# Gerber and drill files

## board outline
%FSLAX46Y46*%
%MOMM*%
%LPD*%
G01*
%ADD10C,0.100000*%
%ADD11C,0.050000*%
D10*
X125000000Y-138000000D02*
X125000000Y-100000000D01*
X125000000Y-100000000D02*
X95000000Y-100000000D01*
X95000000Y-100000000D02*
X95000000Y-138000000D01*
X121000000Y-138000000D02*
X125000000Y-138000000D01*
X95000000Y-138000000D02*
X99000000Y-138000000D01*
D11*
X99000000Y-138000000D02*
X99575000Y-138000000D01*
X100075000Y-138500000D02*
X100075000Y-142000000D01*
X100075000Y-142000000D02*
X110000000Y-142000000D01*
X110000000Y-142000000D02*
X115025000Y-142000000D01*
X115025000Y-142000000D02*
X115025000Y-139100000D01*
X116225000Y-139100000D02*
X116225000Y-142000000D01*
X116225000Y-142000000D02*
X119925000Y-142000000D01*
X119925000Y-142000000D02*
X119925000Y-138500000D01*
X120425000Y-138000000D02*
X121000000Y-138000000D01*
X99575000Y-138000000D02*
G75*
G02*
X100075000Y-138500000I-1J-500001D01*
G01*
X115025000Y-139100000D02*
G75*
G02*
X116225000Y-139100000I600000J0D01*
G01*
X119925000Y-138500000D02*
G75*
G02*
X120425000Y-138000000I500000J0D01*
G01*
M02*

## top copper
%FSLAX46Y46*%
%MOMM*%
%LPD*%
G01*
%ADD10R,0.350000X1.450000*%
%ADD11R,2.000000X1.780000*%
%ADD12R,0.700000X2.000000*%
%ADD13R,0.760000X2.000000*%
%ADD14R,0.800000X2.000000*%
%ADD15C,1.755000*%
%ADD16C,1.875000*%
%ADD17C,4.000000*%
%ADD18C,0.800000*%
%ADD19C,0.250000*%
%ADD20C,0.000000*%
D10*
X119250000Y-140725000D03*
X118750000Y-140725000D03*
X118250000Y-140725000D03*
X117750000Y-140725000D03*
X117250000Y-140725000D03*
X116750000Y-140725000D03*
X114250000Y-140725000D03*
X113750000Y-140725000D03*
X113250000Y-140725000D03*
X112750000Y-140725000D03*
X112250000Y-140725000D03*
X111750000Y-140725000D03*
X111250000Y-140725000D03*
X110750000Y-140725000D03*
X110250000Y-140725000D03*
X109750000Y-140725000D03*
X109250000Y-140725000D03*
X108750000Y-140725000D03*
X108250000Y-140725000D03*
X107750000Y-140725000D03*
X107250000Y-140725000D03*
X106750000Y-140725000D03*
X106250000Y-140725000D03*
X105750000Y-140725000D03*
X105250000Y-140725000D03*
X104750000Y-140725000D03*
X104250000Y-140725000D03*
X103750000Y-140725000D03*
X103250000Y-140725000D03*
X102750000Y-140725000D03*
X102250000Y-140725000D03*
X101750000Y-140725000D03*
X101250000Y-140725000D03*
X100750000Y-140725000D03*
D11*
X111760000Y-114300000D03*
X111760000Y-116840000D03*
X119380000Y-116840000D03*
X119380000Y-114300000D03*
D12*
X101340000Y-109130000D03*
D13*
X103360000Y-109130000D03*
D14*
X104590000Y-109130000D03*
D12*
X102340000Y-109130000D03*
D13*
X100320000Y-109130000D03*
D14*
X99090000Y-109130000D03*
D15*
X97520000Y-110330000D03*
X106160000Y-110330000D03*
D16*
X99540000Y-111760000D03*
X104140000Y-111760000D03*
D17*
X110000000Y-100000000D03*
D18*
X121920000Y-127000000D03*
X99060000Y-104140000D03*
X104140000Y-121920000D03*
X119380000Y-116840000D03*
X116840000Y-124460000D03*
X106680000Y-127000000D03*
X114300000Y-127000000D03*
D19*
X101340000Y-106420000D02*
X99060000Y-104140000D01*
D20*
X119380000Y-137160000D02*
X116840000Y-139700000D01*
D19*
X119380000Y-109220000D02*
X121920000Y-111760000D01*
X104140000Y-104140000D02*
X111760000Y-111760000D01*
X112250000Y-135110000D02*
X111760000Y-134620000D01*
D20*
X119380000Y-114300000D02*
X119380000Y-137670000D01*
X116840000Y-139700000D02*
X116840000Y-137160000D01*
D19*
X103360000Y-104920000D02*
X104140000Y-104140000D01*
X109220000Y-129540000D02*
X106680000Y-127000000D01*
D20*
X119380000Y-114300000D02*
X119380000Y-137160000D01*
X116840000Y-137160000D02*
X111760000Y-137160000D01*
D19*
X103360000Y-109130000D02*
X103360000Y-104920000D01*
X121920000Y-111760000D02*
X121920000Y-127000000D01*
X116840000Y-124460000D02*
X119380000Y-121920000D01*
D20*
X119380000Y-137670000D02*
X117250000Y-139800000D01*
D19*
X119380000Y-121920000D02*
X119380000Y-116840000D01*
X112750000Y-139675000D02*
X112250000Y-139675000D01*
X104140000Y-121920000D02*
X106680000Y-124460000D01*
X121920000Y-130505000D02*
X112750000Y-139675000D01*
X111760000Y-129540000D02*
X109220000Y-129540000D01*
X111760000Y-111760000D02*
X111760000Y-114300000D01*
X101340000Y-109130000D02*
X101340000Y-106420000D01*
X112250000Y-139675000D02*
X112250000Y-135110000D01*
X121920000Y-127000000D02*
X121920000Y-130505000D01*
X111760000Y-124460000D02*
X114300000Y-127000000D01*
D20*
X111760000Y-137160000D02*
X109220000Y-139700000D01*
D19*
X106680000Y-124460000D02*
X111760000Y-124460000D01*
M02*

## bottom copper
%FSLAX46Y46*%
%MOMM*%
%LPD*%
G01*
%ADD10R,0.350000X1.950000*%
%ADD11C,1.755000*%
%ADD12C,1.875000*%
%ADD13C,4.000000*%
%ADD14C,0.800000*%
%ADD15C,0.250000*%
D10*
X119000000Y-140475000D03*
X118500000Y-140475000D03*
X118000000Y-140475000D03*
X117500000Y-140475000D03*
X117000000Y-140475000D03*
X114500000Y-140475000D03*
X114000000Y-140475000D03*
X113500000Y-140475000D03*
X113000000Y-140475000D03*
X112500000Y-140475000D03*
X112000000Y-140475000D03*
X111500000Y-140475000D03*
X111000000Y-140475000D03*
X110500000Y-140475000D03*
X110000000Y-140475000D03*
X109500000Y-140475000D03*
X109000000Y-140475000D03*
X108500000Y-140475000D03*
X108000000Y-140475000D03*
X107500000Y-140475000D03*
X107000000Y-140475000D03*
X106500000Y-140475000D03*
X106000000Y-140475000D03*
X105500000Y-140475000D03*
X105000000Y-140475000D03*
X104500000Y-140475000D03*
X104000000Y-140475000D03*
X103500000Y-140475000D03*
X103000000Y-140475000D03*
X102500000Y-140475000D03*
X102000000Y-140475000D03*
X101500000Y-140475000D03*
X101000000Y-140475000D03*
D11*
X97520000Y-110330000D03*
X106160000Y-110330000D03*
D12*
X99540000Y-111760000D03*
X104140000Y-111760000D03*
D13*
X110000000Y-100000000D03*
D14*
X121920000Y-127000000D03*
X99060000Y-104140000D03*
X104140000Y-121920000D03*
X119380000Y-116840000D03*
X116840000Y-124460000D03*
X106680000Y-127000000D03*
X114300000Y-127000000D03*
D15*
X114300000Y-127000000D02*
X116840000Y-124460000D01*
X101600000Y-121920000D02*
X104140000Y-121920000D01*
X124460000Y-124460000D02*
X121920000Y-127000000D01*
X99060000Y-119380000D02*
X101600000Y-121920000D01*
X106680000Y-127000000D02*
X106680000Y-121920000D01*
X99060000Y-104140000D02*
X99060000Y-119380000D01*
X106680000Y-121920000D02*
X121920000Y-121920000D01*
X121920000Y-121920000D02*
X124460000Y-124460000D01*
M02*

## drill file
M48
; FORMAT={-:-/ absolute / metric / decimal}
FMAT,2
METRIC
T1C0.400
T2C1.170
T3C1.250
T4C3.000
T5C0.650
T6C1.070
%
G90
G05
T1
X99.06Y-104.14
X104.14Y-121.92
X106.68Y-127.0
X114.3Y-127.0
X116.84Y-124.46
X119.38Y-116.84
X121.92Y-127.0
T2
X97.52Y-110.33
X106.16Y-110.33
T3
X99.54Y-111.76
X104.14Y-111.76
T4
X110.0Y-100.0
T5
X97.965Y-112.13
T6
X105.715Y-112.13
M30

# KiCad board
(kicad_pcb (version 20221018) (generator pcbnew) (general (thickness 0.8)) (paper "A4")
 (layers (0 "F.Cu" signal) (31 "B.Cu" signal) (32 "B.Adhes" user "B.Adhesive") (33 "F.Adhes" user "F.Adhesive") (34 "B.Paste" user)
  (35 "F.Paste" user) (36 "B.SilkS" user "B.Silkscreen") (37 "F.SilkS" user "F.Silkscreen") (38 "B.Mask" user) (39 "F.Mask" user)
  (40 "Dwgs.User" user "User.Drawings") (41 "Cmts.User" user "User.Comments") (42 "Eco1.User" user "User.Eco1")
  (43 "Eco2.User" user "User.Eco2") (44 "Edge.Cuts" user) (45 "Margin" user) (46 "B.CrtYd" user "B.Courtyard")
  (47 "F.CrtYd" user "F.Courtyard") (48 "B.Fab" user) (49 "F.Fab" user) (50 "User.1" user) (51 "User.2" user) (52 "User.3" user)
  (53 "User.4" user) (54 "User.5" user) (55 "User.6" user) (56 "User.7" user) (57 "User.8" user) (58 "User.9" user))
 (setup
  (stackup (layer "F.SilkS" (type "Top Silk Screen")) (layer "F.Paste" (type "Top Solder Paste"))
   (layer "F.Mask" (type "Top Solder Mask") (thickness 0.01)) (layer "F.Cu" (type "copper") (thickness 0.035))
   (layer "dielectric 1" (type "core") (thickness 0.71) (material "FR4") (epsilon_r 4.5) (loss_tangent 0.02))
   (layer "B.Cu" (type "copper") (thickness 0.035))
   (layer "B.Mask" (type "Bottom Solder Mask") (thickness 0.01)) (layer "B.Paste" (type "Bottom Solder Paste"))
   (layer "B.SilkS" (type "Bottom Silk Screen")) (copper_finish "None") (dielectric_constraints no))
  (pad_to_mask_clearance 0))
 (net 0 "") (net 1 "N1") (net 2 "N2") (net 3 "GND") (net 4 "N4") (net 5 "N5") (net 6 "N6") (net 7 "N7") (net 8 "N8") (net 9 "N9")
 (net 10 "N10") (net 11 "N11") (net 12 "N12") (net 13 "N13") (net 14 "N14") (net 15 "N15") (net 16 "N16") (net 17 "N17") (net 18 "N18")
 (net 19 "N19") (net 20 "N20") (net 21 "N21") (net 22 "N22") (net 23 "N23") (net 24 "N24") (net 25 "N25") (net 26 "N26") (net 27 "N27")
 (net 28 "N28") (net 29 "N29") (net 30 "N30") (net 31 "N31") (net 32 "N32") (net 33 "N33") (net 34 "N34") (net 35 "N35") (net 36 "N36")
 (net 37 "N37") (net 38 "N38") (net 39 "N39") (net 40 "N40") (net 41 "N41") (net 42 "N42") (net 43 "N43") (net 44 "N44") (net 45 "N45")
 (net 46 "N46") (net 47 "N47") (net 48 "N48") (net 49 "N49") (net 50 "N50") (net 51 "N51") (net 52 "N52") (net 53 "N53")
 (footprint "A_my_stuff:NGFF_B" (layer "F.Cu") (at 110 142)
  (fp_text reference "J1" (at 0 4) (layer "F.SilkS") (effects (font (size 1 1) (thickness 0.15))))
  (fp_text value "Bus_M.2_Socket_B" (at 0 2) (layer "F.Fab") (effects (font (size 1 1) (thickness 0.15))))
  (fp_line (start -11 -4) (end -10.425 -4) (stroke (width 0.05) (type solid)) (layer "Edge.Cuts"))
  (fp_line (start -9.925 -3.5) (end -9.925 0) (stroke (width 0.05) (type solid)) (layer "Edge.Cuts"))
  (fp_line (start -9.925 0) (end 0 0) (stroke (width 0.05) (type solid)) (layer "Edge.Cuts"))
  (fp_line (start 0 0) (end 5.025 0) (stroke (width 0.05) (type solid)) (layer "Edge.Cuts"))
  (fp_line (start 5.025 0) (end 5.025 -2.9) (stroke (width 0.05) (type solid)) (layer "Edge.Cuts"))
  (fp_line (start 6.225 -2.9) (end 6.225 0) (stroke (width 0.05) (type solid)) (layer "Edge.Cuts"))
  (fp_line (start 6.225 0) (end 9.925 0) (stroke (width 0.05) (type solid)) (layer "Edge.Cuts"))
  (fp_line (start 9.925 0) (end 9.925 -3.5) (stroke (width 0.05) (type solid)) (layer "Edge.Cuts"))
  (fp_line (start 10.425 -4) (end 11 -4) (stroke (width 0.05) (type solid)) (layer "Edge.Cuts"))
  (fp_arc (start -10.425 -4) (mid -10.071447 -3.853553) (end -9.925 -3.5) (stroke (width 0.05) (type solid)) (layer "Edge.Cuts"))
  (fp_arc (start 5.025 -2.9) (mid 5.625 -3.5) (end 6.225 -2.9) (stroke (width 0.05) (type solid)) (layer "Edge.Cuts"))
  (fp_arc (start 9.925 -3.5) (mid 10.071447 -3.853553) (end 10.425 -4) (stroke (width 0.05) (type solid)) (layer "Edge.Cuts"))
  (pad "1" smd rect (at 9.25 -1.275) (size 0.35 1.45) (layers "F.Cu") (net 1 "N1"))
  (pad "2" smd rect (at 9 -1.525) (size 0.35 1.95) (layers "B.Cu") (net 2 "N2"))
  (pad "3" smd rect (at 8.75 -1.275) (size 0.35 1.45) (layers "F.Cu") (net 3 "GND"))
  (pad "4" smd rect (at 8.5 -1.525) (size 0.35 1.95) (layers "B.Cu") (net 2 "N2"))
  (pad "5" smd rect (at 8.25 -1.275) (size 0.35 1.45) (layers "F.Cu") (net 3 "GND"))
  (pad "6" smd rect (at 8 -1.525) (size 0.35 1.95) (layers "B.Cu") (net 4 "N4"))
  (pad "7" smd rect (at 7.75 -1.275) (size 0.35 1.45) (layers "F.Cu") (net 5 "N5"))
  (pad "8" smd rect (at 7.5 -1.525) (size 0.35 1.95) (layers "B.Cu") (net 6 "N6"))
  (pad "9" smd rect (at 7.25 -1.275) (size 0.35 1.45) (layers "F.Cu") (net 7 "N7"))
  (pad "10" smd rect (at 7 -1.525) (size 0.35 1.95) (layers "B.Cu") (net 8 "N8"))
  (pad "11" smd rect (at 6.75 -1.275) (size 0.35 1.45) (layers "F.Cu") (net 3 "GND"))
  (pad "20" smd rect (at 4.5 -1.525) (size 0.35 1.95) (layers "B.Cu") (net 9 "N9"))
  (pad "21" smd rect (at 4.25 -1.275) (size 0.35 1.45) (layers "F.Cu") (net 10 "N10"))
  (pad "22" smd rect (at 4 -1.525) (size 0.35 1.95) (layers "B.Cu") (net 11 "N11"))
  (pad "23" smd rect (at 3.75 -1.275) (size 0.35 1.45) (layers "F.Cu") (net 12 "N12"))
  (pad "24" smd rect (at 3.5 -1.525) (size 0.35 1.95) (layers "B.Cu") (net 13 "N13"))
  (pad "25" smd rect (at 3.25 -1.275) (size 0.35 1.45) (layers "F.Cu") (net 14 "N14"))
  (pad "26" smd rect (at 3 -1.525) (size 0.35 1.95) (layers "B.Cu") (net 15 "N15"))
  (pad "27" smd rect (at 2.75 -1.275) (size 0.35 1.45) (layers "F.Cu") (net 3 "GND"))
  (pad "28" smd rect (at 2.5 -1.525) (size 0.35 1.95) (layers "B.Cu") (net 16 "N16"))
  (pad "29" smd rect (at 2.25 -1.275) (size 0.35 1.45) (layers "F.Cu") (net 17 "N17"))
  (pad "30" smd rect (at 2 -1.525) (size 0.35 1.95) (layers "B.Cu") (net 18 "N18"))
  (pad "31" smd rect (at 1.75 -1.275) (size 0.35 1.45) (layers "F.Cu") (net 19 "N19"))
  (pad "32" smd rect (at 1.5 -1.525) (size 0.35 1.95) (layers "B.Cu") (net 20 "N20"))
  (pad "33" smd rect (at 1.25 -1.275) (size 0.35 1.45) (layers "F.Cu") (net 3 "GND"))
  (pad "34" smd rect (at 1 -1.525) (size 0.35 1.95) (layers "B.Cu") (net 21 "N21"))
  (pad "35" smd rect (at 0.75 -1.275) (size 0.35 1.45) (layers "F.Cu") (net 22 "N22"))
  (pad "36" smd rect (at 0.5 -1.525) (size 0.35 1.95) (layers "B.Cu") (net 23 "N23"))
  (pad "37" smd rect (at 0.25 -1.275) (size 0.35 1.45) (layers "F.Cu") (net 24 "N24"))
  (pad "38" smd rect (at 0 -1.525) (size 0.35 1.95) (layers "B.Cu") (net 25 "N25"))
  (pad "39" smd rect (at -0.25 -1.275) (size 0.35 1.45) (layers "F.Cu") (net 3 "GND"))
  (pad "40" smd rect (at -0.5 -1.525) (size 0.35 1.95) (layers "B.Cu") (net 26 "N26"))
  (pad "41" smd rect (at -0.75 -1.275) (size 0.35 1.45) (layers "F.Cu") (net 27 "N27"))
  (pad "42" smd rect (at -1 -1.525) (size 0.35 1.95) (layers "B.Cu") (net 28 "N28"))
  (pad "43" smd rect (at -1.25 -1.275) (size 0.35 1.45) (layers "F.Cu") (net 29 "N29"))
  (pad "44" smd rect (at -1.5 -1.525) (size 0.35 1.95) (layers "B.Cu") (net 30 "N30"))
  (pad "45" smd rect (at -1.75 -1.275) (size 0.35 1.45) (layers "F.Cu") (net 3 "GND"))
  (pad "46" smd rect (at -2 -1.525) (size 0.35 1.95) (layers "B.Cu") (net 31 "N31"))
  (pad "47" smd rect (at -2.25 -1.275) (size 0.35 1.45) (layers "F.Cu") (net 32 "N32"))
  (pad "48" smd rect (at -2.5 -1.525) (size 0.35 1.95) (layers "B.Cu") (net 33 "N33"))
  (pad "49" smd rect (at -2.75 -1.275) (size 0.35 1.45) (layers "F.Cu") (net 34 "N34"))
  (pad "50" smd rect (at -3 -1.525) (size 0.35 1.95) (layers "B.Cu") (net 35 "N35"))
  (pad "51" smd rect (at -3.25 -1.275) (size 0.35 1.45) (layers "F.Cu") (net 3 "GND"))
  (pad "52" smd rect (at -3.5 -1.525) (size 0.35 1.95) (layers "B.Cu") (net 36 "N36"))
  (pad "53" smd rect (at -3.75 -1.275) (size 0.35 1.45) (layers "F.Cu") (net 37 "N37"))
  (pad "54" smd rect (at -4 -1.525) (size 0.35 1.95) (layers "B.Cu") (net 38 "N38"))
  (pad "55" smd rect (at -4.25 -1.275) (size 0.35 1.45) (layers "F.Cu") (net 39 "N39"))
  (pad "56" smd rect (at -4.5 -1.525) (size 0.35 1.95) (layers "B.Cu") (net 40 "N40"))
  (pad "57" smd rect (at -4.75 -1.275) (size 0.35 1.45) (layers "F.Cu") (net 3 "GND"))
  (pad "58" smd rect (at -5 -1.525) (size 0.35 1.95) (layers "B.Cu") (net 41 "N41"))
  (pad "59" smd rect (at -5.25 -1.275) (size 0.35 1.45) (layers "F.Cu") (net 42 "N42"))
  (pad "60" smd rect (at -5.5 -1.525) (size 0.35 1.95) (layers "B.Cu") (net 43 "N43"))
  (pad "61" smd rect (at -5.75 -1.275) (size 0.35 1.45) (layers "F.Cu") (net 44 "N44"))
  (pad "62" smd rect (at -6 -1.525) (size 0.35 1.95) (layers "B.Cu") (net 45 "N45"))
  (pad "63" smd rect (at -6.25 -1.275) (size 0.35 1.45) (layers "F.Cu") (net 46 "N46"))
  (pad "64" smd rect (at -6.5 -1.525) (size 0.35 1.95) (layers "B.Cu") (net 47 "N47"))
  (pad "65" smd rect (at -6.75 -1.275) (size 0.35 1.45) (layers "F.Cu") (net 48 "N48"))
  (pad "66" smd rect (at -7 -1.525) (size 0.35 1.95) (layers "B.Cu") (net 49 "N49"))
  (pad "67" smd rect (at -7.25 -1.275) (size 0.35 1.45) (layers "F.Cu") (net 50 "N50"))
  (pad "68" smd rect (at -7.5 -1.525) (size 0.35 1.95) (layers "B.Cu") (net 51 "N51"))
  (pad "69" smd rect (at -7.75 -1.275) (size 0.35 1.45) (layers "F.Cu") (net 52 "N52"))
  (pad "70" smd rect (at -8 -1.525) (size 0.35 1.95) (layers "B.Cu") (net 2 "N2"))
  (pad "71" smd rect (at -8.25 -1.275) (size 0.35 1.45) (layers "F.Cu") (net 3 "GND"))
  (pad "72" smd rect (at -8.5 -1.525) (size 0.35 1.95) (layers "B.Cu") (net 2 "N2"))
  (pad "73" smd rect (at -8.75 -1.275) (size 0.35 1.45) (layers "F.Cu") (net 3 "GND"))
  (pad "74" smd rect (at -9 -1.525) (size 0.35 1.95) (layers "B.Cu") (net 2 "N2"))
  (pad "75" smd rect (at -9.25 -1.275) (size 0.35 1.45) (layers "F.Cu") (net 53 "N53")))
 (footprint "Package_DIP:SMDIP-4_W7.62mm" (layer "F.Cu") (at 115.57 115.57)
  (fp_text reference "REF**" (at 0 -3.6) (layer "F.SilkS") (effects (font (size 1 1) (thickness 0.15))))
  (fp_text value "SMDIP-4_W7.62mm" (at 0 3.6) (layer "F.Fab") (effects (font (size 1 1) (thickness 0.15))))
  (pad "1" smd rect (at -3.81 -1.27) (size 2 1.78) (layers "F.Cu" "F.Paste" "F.Mask"))
  (pad "2" smd rect (at -3.81 1.27) (size 2 1.78) (layers "F.Cu" "F.Paste" "F.Mask"))
  (pad "3" smd rect (at 3.81 1.27) (size 2 1.78) (layers "F.Cu" "F.Paste" "F.Mask"))
  (pad "4" smd rect (at 3.81 -1.27) (size 2 1.78) (layers "F.Cu" "F.Paste" "F.Mask")))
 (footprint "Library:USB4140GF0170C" (layer "F.Cu") (at 101.84 110.58)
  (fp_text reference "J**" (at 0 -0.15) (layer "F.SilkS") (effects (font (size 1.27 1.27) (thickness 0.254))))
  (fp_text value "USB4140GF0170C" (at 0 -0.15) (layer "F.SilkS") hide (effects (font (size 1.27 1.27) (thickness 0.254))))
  (pad "" np_thru_hole circle (at -3.875 1.55) (size 0.65 0.65) (drill 0.65) (layers "*.Cu" "*.Mask"))
  (pad "" np_thru_hole circle (at 3.875 1.55) (size 1.07 1.07) (drill 1.07) (layers "*.Cu" "*.Mask"))
  (pad "A5" smd rect (at -0.5 -1.45) (size 0.7 2) (layers "F.Cu" "F.Paste" "F.Mask"))
  (pad "A9" smd rect (at 1.52 -1.45) (size 0.76 2) (layers "F.Cu" "F.Paste" "F.Mask"))
  (pad "A12" smd rect (at 2.75 -1.45) (size 0.8 2) (layers "F.Cu" "F.Paste" "F.Mask"))
  (pad "B5" smd rect (at 0.5 -1.45) (size 0.7 2) (layers "F.Cu" "F.Paste" "F.Mask"))
  (pad "B9" smd rect (at -1.52 -1.45) (size 0.76 2) (layers "F.Cu" "F.Paste" "F.Mask"))
  (pad "B12" smd rect (at -2.75 -1.45) (size 0.8 2) (layers "F.Cu" "F.Paste" "F.Mask"))
  (pad "MH1" thru_hole circle (at -4.32 -0.25) (size 1.755 1.755) (drill 1.17) (layers "*.Cu" "*.Mask"))
  (pad "MH2" thru_hole circle (at 4.32 -0.25) (size 1.755 1.755) (drill 1.17) (layers "*.Cu" "*.Mask"))
  (pad "MH3" thru_hole circle (at -2.3 1.18) (size 1.875 1.875) (drill 1.25) (layers "*.Cu" "*.Mask"))
  (pad "MH4" thru_hole circle (at 2.3 1.18) (size 1.875 1.875) (drill 1.25) (layers "*.Cu" "*.Mask")))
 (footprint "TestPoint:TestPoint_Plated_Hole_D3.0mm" (layer "F.Cu") (at 110 100)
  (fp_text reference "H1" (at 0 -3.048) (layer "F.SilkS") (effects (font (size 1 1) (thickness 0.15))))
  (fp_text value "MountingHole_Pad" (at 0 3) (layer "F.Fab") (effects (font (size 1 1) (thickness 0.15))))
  (pad "1" thru_hole circle (at 0 0) (size 4 4) (drill 3) (layers "*.Cu" "*.Mask") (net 3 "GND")))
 (gr_line (start 125 138) (end 125 100) (stroke (width 0.1) (type default)) (layer "Edge.Cuts"))
 (gr_line (start 125 100) (end 95 100) (stroke (width 0.1) (type default)) (layer "Edge.Cuts"))
 (gr_line (start 95 100) (end 95 138) (stroke (width 0.1) (type default)) (layer "Edge.Cuts"))
 (gr_line (start 121 138) (end 125 138) (stroke (width 0.1) (type default)) (layer "Edge.Cuts"))
 (gr_line (start 95 138) (end 99 138) (stroke (width 0.1) (type default)) (layer "Edge.Cuts"))
 (segment (start 101.34 106.42) (end 99.06 104.14) (width 0.25) (layer "F.Cu") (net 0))
 (segment (start 119.38 137.16) (end 116.84 139.7) (width 0) (layer "F.Cu") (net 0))
 (segment (start 119.38 109.22) (end 121.92 111.76) (width 0.25) (layer "F.Cu") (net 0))
 (segment (start 104.14 104.14) (end 111.76 111.76) (width 0.25) (layer "F.Cu") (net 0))
 (segment (start 112.25 135.11) (end 111.76 134.62) (width 0.25) (layer "F.Cu") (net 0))
 (segment (start 119.38 114.3) (end 119.38 137.67) (width 0) (layer "F.Cu") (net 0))
 (segment (start 116.84 139.7) (end 116.84 137.16) (width 0) (layer "F.Cu") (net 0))
 (segment (start 103.36 104.92) (end 104.14 104.14) (width 0.25) (layer "F.Cu") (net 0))
 (segment (start 109.22 129.54) (end 106.68 127) (width 0.25) (layer "F.Cu") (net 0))
 (segment (start 119.38 114.3) (end 119.38 137.16) (width 0) (layer "F.Cu") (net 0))
 (segment (start 116.84 137.16) (end 111.76 137.16) (width 0) (layer "F.Cu") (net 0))
 (segment (start 103.36 109.13) (end 103.36 104.92) (width 0.25) (layer "F.Cu") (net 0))
 (segment (start 121.92 111.76) (end 121.92 127) (width 0.25) (layer "F.Cu") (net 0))
 (segment (start 116.84 124.46) (end 119.38 121.92) (width 0.25) (layer "F.Cu") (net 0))
 (segment (start 119.38 137.67) (end 117.25 139.8) (width 0) (layer "F.Cu") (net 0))
 (segment (start 119.38 121.92) (end 119.38 116.84) (width 0.25) (layer "F.Cu") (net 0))
 (segment (start 112.75 139.675) (end 112.25 139.675) (width 0.25) (layer "F.Cu") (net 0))
 (segment (start 104.14 121.92) (end 106.68 124.46) (width 0.25) (layer "F.Cu") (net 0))
 (segment (start 121.92 130.505) (end 112.75 139.675) (width 0.25) (layer "F.Cu") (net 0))
 (segment (start 111.76 129.54) (end 109.22 129.54) (width 0.25) (layer "F.Cu") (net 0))
 (segment (start 111.76 111.76) (end 111.76 114.3) (width 0.25) (layer "F.Cu") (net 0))
 (segment (start 101.34 109.13) (end 101.34 106.42) (width 0.25) (layer "F.Cu") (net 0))
 (segment (start 112.25 139.675) (end 112.25 135.11) (width 0.25) (layer "F.Cu") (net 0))
 (segment (start 121.92 127) (end 121.92 130.505) (width 0.25) (layer "F.Cu") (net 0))
 (segment (start 111.76 124.46) (end 114.3 127) (width 0.25) (layer "F.Cu") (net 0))
 (segment (start 111.76 137.16) (end 109.22 139.7) (width 0) (layer "F.Cu") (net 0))
 (segment (start 106.68 124.46) (end 111.76 124.46) (width 0.25) (layer "F.Cu") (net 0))
 (via (at 121.92 127) (size 0.8) (drill 0.4) (layers "F.Cu" "B.Cu") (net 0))
 (via (at 99.06 104.14) (size 0.8) (drill 0.4) (layers "F.Cu" "B.Cu") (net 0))
 (via (at 104.14 121.92) (size 0.8) (drill 0.4) (layers "F.Cu" "B.Cu") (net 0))
 (via (at 119.38 116.84) (size 0.8) (drill 0.4) (layers "F.Cu" "B.Cu") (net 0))
 (via (at 116.84 124.46) (size 0.8) (drill 0.4) (layers "F.Cu" "B.Cu") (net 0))
 (via (at 106.68 127) (size 0.8) (drill 0.4) (layers "F.Cu" "B.Cu") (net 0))
 (via (at 114.3 127) (size 0.8) (drill 0.4) (layers "F.Cu" "B.Cu") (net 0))
 (segment (start 114.3 127) (end 116.84 124.46) (width 0.25) (layer "B.Cu") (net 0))
 (segment (start 101.6 121.92) (end 104.14 121.92) (width 0.25) (layer "B.Cu") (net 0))
 (segment (start 124.46 124.46) (end 121.92 127) (width 0.25) (layer "B.Cu") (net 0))
 (segment (start 99.06 119.38) (end 101.6 121.92) (width 0.25) (layer "B.Cu") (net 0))
 (segment (start 106.68 127) (end 106.68 121.92) (width 0.25) (layer "B.Cu") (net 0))
 (segment (start 99.06 104.14) (end 99.06 119.38) (width 0.25) (layer "B.Cu") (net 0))
 (segment (start 106.68 121.92) (end 121.92 121.92) (width 0.25) (layer "B.Cu") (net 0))
 (segment (start 121.92 121.92) (end 124.46 124.46) (width 0.25) (layer "B.Cu") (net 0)))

